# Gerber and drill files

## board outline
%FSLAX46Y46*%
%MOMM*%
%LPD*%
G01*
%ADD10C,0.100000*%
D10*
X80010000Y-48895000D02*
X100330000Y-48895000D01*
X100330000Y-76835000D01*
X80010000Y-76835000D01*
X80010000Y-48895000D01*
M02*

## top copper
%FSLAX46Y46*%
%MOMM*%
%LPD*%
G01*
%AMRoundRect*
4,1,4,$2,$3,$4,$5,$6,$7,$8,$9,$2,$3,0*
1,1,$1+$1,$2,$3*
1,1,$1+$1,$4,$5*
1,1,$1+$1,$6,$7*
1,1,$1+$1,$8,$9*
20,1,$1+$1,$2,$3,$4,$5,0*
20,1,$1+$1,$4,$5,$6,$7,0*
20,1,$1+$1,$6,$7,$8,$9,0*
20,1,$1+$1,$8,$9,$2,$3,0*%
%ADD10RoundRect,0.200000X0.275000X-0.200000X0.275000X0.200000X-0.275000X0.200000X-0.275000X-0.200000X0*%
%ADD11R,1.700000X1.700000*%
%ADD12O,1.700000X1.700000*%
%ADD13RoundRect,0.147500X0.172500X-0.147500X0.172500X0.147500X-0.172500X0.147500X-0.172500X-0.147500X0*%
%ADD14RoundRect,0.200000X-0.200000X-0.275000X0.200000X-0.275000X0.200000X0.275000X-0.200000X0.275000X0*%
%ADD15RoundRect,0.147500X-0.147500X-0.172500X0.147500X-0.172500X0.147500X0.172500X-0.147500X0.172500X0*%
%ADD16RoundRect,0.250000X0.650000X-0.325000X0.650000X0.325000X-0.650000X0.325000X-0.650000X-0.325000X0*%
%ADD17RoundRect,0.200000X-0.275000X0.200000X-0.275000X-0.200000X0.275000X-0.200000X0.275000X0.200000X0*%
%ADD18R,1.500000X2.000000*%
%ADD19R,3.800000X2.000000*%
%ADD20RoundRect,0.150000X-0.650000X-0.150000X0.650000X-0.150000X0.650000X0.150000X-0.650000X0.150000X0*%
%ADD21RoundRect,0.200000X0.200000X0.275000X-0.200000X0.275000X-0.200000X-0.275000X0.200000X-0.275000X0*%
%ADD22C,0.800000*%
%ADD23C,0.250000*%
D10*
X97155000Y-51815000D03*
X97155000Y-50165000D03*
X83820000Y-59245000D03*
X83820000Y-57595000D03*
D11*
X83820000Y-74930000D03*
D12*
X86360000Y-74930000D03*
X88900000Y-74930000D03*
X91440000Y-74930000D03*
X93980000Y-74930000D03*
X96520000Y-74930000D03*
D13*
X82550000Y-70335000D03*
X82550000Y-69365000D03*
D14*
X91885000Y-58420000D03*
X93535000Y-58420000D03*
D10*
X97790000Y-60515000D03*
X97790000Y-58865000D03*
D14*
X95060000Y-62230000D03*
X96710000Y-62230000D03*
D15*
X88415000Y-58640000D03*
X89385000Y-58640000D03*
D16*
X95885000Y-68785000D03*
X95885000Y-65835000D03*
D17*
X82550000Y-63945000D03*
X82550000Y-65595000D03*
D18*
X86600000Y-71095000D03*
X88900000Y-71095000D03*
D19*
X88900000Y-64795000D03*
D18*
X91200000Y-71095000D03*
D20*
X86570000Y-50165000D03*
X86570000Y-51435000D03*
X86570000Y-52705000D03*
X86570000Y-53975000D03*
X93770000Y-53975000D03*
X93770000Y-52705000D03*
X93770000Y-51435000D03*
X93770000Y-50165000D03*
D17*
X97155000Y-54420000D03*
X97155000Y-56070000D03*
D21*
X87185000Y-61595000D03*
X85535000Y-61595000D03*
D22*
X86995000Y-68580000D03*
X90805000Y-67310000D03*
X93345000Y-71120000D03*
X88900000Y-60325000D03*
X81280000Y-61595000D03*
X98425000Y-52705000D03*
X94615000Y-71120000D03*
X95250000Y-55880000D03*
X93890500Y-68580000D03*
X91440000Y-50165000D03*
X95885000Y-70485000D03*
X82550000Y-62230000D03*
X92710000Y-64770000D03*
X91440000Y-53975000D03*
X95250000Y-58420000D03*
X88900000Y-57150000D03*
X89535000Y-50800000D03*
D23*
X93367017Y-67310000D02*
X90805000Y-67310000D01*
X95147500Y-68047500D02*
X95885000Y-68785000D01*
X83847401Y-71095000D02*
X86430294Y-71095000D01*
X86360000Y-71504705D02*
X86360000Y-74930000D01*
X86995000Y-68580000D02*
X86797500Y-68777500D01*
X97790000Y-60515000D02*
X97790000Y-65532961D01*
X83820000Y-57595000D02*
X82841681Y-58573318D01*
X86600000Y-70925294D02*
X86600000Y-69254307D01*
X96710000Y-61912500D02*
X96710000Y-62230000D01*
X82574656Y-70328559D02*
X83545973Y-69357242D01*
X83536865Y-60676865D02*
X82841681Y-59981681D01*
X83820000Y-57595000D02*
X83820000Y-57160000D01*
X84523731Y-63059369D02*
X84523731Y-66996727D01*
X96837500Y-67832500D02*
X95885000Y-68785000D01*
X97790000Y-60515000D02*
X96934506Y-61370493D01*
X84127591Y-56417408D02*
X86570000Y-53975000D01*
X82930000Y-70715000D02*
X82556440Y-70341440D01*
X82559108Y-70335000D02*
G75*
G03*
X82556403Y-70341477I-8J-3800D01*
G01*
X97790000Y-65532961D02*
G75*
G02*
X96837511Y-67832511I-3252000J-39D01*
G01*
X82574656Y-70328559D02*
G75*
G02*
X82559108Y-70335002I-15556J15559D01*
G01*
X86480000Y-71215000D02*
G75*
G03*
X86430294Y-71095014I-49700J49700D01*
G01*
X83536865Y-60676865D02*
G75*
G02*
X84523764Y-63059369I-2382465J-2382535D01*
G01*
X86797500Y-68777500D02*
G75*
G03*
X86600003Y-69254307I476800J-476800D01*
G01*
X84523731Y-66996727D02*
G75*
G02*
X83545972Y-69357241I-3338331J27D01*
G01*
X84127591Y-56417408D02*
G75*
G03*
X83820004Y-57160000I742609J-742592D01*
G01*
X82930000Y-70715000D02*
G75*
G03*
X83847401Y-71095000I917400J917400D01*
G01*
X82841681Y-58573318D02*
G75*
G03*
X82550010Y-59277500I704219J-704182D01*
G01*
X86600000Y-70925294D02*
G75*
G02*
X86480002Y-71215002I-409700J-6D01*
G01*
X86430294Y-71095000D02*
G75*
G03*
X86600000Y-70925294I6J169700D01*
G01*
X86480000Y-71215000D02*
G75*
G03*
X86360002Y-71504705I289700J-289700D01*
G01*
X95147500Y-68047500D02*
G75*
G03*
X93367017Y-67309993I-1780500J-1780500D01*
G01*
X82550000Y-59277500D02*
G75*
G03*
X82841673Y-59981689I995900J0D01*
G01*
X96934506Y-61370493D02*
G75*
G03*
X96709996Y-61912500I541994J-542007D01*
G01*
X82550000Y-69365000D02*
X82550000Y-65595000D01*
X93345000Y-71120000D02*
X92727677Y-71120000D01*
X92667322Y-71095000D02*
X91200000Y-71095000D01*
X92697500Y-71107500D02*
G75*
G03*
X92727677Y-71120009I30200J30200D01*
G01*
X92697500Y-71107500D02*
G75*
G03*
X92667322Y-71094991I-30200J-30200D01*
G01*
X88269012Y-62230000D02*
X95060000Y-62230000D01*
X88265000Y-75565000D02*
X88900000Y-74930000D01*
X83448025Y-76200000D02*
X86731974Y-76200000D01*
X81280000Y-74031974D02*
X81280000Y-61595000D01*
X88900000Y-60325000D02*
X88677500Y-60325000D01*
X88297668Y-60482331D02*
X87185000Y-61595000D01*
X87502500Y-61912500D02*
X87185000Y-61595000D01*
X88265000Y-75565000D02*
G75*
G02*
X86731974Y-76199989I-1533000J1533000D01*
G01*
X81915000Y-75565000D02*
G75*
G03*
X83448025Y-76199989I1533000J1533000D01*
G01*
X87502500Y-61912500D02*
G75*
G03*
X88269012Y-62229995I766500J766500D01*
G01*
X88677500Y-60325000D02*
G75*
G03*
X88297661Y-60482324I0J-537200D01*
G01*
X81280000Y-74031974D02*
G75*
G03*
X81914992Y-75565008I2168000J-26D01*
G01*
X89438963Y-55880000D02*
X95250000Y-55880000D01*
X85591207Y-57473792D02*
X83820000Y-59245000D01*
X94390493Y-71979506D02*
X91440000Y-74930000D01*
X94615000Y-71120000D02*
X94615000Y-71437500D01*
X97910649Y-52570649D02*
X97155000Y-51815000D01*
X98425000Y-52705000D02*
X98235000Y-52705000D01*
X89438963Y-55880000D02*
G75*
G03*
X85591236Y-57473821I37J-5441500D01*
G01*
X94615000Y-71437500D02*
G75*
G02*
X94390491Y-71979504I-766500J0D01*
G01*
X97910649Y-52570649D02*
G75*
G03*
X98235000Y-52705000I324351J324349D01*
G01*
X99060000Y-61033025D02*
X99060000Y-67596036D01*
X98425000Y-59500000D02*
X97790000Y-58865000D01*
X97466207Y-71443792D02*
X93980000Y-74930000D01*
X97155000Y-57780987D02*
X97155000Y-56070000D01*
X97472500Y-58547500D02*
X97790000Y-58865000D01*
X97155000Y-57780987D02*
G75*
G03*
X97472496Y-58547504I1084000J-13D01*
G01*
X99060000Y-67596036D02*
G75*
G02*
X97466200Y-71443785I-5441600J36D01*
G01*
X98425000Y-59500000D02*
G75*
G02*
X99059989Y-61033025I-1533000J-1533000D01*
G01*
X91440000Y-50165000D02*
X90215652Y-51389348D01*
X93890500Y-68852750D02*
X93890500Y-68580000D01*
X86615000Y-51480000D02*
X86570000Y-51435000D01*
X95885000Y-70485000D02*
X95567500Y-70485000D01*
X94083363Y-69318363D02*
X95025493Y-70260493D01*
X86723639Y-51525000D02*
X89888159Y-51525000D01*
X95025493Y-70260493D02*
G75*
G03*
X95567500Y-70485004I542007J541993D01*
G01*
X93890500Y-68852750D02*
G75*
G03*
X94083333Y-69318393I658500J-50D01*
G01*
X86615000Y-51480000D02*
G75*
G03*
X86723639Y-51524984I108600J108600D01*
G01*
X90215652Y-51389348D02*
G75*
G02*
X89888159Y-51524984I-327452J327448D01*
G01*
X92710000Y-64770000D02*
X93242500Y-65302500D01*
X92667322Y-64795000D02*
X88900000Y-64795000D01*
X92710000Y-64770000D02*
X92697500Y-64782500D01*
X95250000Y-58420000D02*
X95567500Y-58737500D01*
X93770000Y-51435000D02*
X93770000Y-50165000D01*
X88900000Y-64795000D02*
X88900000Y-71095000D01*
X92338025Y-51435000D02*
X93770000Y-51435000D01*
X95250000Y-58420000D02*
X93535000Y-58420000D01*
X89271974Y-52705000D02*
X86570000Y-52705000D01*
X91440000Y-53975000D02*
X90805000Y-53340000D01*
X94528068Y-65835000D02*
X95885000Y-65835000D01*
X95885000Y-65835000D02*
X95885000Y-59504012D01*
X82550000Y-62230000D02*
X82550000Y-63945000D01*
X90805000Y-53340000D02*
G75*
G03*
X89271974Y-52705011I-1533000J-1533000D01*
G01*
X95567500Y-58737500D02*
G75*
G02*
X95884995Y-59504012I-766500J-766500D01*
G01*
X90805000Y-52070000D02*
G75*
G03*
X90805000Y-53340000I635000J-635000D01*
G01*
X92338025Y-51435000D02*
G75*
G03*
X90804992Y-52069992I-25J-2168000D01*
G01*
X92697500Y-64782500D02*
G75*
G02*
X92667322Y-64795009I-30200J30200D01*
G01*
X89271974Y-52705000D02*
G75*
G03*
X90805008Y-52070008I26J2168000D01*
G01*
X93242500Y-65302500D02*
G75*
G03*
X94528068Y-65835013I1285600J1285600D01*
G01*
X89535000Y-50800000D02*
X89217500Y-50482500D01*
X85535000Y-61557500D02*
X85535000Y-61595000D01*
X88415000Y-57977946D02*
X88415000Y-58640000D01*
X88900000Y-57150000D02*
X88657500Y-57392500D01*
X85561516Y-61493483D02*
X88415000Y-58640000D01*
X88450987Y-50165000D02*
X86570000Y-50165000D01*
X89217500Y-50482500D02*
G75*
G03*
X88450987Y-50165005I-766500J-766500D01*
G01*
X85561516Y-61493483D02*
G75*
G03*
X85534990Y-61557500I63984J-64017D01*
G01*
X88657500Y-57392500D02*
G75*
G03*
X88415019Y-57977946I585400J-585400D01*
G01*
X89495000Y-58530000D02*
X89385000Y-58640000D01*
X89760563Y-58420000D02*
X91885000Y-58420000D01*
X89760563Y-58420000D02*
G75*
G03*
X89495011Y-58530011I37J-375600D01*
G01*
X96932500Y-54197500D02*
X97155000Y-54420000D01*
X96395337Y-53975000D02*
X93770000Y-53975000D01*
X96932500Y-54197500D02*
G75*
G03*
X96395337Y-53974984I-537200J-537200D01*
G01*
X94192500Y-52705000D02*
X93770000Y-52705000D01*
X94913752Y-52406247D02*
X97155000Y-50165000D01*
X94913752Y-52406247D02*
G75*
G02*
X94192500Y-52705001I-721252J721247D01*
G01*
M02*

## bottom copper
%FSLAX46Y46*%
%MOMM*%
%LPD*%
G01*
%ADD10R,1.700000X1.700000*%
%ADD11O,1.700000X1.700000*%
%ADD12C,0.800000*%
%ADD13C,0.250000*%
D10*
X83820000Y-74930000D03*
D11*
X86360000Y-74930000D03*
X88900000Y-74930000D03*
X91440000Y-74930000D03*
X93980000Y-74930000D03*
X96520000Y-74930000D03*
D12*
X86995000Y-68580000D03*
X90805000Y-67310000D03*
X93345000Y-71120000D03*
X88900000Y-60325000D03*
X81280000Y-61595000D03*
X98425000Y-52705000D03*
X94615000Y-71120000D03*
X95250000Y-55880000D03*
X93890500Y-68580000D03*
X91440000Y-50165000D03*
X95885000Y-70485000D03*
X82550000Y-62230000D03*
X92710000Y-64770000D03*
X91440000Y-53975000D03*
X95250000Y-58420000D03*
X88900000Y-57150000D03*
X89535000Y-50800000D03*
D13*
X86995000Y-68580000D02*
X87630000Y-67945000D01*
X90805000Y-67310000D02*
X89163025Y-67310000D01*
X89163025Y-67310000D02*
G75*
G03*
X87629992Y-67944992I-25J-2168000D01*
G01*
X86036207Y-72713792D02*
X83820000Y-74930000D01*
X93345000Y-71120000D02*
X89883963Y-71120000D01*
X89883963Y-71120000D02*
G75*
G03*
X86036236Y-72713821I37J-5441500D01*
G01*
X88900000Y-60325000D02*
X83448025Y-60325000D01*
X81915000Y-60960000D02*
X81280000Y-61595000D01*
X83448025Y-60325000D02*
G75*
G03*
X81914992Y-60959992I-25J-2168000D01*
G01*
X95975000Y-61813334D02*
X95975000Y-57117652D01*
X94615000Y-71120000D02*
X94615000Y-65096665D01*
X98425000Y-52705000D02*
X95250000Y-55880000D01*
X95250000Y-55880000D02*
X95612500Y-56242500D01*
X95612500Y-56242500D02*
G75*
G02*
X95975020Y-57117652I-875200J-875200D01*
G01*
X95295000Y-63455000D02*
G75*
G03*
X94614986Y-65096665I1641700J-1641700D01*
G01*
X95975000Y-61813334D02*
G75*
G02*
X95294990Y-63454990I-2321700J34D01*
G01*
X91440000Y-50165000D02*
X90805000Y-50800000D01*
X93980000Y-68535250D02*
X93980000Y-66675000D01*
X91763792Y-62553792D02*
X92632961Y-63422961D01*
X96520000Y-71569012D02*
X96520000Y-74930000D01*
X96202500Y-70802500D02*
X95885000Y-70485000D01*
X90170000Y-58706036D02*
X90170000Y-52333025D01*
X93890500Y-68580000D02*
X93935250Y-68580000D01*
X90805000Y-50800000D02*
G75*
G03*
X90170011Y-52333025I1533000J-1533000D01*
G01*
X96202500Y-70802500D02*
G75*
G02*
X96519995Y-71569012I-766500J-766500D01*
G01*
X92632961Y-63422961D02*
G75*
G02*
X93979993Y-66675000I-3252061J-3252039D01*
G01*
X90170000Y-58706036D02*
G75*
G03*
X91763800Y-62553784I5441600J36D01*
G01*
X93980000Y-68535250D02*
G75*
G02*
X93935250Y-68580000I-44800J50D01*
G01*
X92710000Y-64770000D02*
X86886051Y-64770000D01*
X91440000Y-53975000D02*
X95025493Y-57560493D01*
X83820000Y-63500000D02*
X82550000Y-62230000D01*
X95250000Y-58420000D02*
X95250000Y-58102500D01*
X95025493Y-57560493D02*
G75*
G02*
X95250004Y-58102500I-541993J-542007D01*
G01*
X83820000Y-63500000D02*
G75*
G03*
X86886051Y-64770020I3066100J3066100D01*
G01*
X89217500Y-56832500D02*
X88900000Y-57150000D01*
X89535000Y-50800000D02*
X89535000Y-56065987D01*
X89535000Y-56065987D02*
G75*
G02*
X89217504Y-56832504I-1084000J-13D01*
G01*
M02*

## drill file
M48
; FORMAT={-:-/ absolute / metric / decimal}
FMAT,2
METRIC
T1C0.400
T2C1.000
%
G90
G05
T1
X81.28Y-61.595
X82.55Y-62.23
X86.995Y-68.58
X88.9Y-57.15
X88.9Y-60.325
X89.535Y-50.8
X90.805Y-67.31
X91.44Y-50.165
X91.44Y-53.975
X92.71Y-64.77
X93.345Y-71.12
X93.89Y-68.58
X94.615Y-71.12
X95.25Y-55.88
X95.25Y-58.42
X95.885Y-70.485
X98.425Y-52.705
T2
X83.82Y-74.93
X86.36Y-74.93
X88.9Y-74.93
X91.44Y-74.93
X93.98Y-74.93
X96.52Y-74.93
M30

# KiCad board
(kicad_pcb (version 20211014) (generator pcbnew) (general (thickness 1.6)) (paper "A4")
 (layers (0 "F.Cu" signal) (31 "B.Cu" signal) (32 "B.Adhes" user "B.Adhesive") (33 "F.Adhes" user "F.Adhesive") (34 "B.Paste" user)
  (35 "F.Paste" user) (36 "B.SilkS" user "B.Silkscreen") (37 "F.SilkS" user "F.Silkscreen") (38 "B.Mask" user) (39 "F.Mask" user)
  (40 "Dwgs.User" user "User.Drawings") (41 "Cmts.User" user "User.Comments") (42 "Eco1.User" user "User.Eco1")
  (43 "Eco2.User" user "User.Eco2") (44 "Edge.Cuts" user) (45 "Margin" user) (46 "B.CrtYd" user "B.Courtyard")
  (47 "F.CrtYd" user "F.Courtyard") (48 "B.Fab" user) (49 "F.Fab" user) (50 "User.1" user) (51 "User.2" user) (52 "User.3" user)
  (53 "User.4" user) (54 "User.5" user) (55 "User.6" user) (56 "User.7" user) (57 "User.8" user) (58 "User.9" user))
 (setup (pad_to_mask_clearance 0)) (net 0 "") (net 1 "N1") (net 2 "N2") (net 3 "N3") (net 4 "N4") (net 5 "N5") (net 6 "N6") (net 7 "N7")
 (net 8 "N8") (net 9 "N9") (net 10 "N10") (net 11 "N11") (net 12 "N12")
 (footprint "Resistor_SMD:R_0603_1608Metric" (layer "F.Cu") (at 97.155 50.99 90)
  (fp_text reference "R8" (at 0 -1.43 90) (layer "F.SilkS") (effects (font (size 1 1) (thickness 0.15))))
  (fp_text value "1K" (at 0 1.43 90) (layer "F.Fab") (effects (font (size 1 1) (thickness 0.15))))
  (pad "1" smd roundrect (at -0.825 0 90) (size 0.8 0.95) (layers "F.Cu" "F.Paste" "F.Mask") (roundrect_rratio 0.25) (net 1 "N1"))
  (pad "2" smd roundrect (at 0.825 0 90) (size 0.8 0.95) (layers "F.Cu" "F.Paste" "F.Mask") (roundrect_rratio 0.25) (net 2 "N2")))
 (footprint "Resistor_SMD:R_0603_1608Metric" (layer "F.Cu") (at 83.82 58.42 90)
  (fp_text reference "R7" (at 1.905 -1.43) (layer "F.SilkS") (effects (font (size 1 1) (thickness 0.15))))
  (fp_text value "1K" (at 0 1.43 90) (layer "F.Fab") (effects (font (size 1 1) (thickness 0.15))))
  (pad "1" smd roundrect (at -0.825 0 90) (size 0.8 0.95) (layers "F.Cu" "F.Paste" "F.Mask") (roundrect_rratio 0.25) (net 1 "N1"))
  (pad "2" smd roundrect (at 0.825 0 90) (size 0.8 0.95) (layers "F.Cu" "F.Paste" "F.Mask") (roundrect_rratio 0.25) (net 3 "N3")))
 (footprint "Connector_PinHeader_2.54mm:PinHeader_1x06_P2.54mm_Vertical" (layer "F.Cu") (at 83.82 74.93 90)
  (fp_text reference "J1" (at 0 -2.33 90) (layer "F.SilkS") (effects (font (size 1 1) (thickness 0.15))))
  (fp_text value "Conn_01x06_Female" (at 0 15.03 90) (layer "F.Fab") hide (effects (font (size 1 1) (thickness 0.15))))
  (pad "1" thru_hole rect (at 0 0 90) (size 1.7 1.7) (drill 1) (layers *.Cu *.Mask) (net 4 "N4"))
  (pad "2" thru_hole oval (at 0 2.54 90) (size 1.7 1.7) (drill 1) (layers *.Cu *.Mask) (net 3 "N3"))
  (pad "3" thru_hole oval (at 0 5.08 90) (size 1.7 1.7) (drill 1) (layers *.Cu *.Mask) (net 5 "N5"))
  (pad "4" thru_hole oval (at 0 7.62 90) (size 1.7 1.7) (drill 1) (layers *.Cu *.Mask) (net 1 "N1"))
  (pad "5" thru_hole oval (at 0 10.16 90) (size 1.7 1.7) (drill 1) (layers *.Cu *.Mask) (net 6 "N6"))
  (pad "6" thru_hole oval (at 0 12.7 90) (size 1.7 1.7) (drill 1) (layers *.Cu *.Mask) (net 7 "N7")))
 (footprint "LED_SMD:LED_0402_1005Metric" (layer "F.Cu") (at 82.55 69.85 90)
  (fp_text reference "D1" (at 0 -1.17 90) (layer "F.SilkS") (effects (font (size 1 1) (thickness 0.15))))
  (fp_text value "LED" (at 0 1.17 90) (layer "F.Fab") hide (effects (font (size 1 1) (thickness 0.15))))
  (pad "1" smd roundrect (at -0.485 0 90) (size 0.59 0.64) (layers "F.Cu" "F.Paste" "F.Mask") (roundrect_rratio 0.25) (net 3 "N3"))
  (pad "2" smd roundrect (at 0.485 0 90) (size 0.59 0.64) (layers "F.Cu" "F.Paste" "F.Mask") (roundrect_rratio 0.25) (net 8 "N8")))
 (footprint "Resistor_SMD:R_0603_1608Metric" (layer "F.Cu") (at 92.71 58.42)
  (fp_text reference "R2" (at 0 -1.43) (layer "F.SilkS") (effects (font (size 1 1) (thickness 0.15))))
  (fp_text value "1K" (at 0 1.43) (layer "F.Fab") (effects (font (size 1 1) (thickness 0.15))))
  (pad "1" smd roundrect (at -0.825 0) (size 0.8 0.95) (layers "F.Cu" "F.Paste" "F.Mask") (roundrect_rratio 0.25) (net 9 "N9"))
  (pad "2" smd roundrect (at 0.825 0) (size 0.8 0.95) (layers "F.Cu" "F.Paste" "F.Mask") (roundrect_rratio 0.25) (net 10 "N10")))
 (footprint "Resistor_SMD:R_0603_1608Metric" (layer "F.Cu") (at 97.79 59.69 90)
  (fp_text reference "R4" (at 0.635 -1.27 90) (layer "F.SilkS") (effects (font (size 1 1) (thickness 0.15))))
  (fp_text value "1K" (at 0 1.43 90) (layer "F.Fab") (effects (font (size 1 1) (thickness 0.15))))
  (pad "1" smd roundrect (at -0.825 0 90) (size 0.8 0.95) (layers "F.Cu" "F.Paste" "F.Mask") (roundrect_rratio 0.25) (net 3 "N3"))
  (pad "2" smd roundrect (at 0.825 0 90) (size 0.8 0.95) (layers "F.Cu" "F.Paste" "F.Mask") (roundrect_rratio 0.25) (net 6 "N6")))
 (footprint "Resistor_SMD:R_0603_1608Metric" (layer "F.Cu") (at 95.885 62.23)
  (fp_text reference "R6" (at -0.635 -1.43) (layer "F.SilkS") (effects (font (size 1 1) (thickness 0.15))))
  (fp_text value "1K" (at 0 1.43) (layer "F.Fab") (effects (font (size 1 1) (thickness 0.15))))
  (pad "1" smd roundrect (at -0.825 0) (size 0.8 0.95) (layers "F.Cu" "F.Paste" "F.Mask") (roundrect_rratio 0.25) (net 5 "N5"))
  (pad "2" smd roundrect (at 0.825 0) (size 0.8 0.95) (layers "F.Cu" "F.Paste" "F.Mask") (roundrect_rratio 0.25) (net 3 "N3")))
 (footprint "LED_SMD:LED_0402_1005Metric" (layer "F.Cu") (at 88.9 58.64)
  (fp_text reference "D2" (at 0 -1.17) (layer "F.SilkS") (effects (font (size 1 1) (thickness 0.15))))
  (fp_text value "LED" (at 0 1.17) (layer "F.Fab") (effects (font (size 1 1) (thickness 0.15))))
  (pad "1" smd roundrect (at -0.485 0) (size 0.59 0.64) (layers "F.Cu" "F.Paste" "F.Mask") (roundrect_rratio 0.25) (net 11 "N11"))
  (pad "2" smd roundrect (at 0.485 0) (size 0.59 0.64) (layers "F.Cu" "F.Paste" "F.Mask") (roundrect_rratio 0.25) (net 9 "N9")))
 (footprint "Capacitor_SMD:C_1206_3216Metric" (layer "F.Cu") (at 95.885 67.31 90)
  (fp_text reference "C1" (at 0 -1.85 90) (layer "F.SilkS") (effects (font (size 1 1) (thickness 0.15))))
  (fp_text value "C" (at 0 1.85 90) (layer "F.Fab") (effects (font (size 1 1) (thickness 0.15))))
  (pad "1" smd roundrect (at -1.475 0 90) (size 1.15 1.8) (layers "F.Cu" "F.Paste" "F.Mask") (roundrect_rratio 0.2173913043) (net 3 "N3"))
  (pad "2" smd roundrect (at 1.475 0 90) (size 1.15 1.8) (layers "F.Cu" "F.Paste" "F.Mask") (roundrect_rratio 0.2173913043) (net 10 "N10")))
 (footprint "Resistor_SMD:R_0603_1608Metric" (layer "F.Cu") (at 82.55 64.77 -90)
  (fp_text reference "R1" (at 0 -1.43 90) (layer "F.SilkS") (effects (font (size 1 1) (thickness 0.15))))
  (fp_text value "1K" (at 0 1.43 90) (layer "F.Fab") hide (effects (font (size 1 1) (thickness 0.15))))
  (pad "1" smd roundrect (at -0.825 0 270) (size 0.8 0.95) (layers "F.Cu" "F.Paste" "F.Mask") (roundrect_rratio 0.25) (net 10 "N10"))
  (pad "2" smd roundrect (at 0.825 0 270) (size 0.8 0.95) (layers "F.Cu" "F.Paste" "F.Mask") (roundrect_rratio 0.25) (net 8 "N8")))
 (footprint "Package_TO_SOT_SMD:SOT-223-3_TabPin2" (layer "F.Cu") (at 88.9 67.945 90)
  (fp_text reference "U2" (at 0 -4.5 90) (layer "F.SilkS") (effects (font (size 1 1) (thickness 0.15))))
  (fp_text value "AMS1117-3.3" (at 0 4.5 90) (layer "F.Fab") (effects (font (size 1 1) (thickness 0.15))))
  (pad "1" smd rect (at -3.15 -2.3 90) (size 2 1.5) (layers "F.Cu" "F.Paste" "F.Mask") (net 3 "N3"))
  (pad "2" smd rect (at -3.15 0 90) (size 2 1.5) (layers "F.Cu" "F.Paste" "F.Mask") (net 10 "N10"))
  (pad "2" smd rect (at 3.15 0 90) (size 2 3.8) (layers "F.Cu" "F.Paste" "F.Mask") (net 10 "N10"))
  (pad "3" smd rect (at -3.15 2.3 90) (size 2 1.5) (layers "F.Cu" "F.Paste" "F.Mask") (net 4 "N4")))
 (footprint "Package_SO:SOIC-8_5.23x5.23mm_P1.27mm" (layer "F.Cu") (at 90.17 52.07)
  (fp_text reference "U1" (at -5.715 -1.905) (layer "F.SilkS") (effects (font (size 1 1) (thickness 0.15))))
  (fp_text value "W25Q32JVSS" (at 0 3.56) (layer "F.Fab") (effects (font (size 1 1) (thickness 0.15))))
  (pad "1" smd roundrect (at -3.6 -1.905) (size 1.6 0.6) (layers "F.Cu" "F.Paste" "F.Mask") (roundrect_rratio 0.25) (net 11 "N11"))
  (pad "2" smd roundrect (at -3.6 -0.635) (size 1.6 0.6) (layers "F.Cu" "F.Paste" "F.Mask") (roundrect_rratio 0.25) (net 7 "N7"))
  (pad "3" smd roundrect (at -3.6 0.635) (size 1.6 0.6) (layers "F.Cu" "F.Paste" "F.Mask") (roundrect_rratio 0.25) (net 10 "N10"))
  (pad "4" smd roundrect (at -3.6 1.905) (size 1.6 0.6) (layers "F.Cu" "F.Paste" "F.Mask") (roundrect_rratio 0.25) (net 3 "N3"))
  (pad "5" smd roundrect (at 3.6 1.905) (size 1.6 0.6) (layers "F.Cu" "F.Paste" "F.Mask") (roundrect_rratio 0.25) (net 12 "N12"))
  (pad "6" smd roundrect (at 3.6 0.635) (size 1.6 0.6) (layers "F.Cu" "F.Paste" "F.Mask") (roundrect_rratio 0.25) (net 2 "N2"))
  (pad "7" smd roundrect (at 3.6 -0.635) (size 1.6 0.6) (layers "F.Cu" "F.Paste" "F.Mask") (roundrect_rratio 0.25) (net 10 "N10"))
  (pad "8" smd roundrect (at 3.6 -1.905) (size 1.6 0.6) (layers "F.Cu" "F.Paste" "F.Mask") (roundrect_rratio 0.25) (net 10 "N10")))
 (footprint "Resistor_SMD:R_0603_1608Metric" (layer "F.Cu") (at 97.155 55.245 -90)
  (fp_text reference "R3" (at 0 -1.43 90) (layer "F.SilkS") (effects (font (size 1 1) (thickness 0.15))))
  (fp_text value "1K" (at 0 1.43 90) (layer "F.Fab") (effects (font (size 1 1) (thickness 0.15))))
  (pad "1" smd roundrect (at -0.825 0 270) (size 0.8 0.95) (layers "F.Cu" "F.Paste" "F.Mask") (roundrect_rratio 0.25) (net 12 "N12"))
  (pad "2" smd roundrect (at 0.825 0 270) (size 0.8 0.95) (layers "F.Cu" "F.Paste" "F.Mask") (roundrect_rratio 0.25) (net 6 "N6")))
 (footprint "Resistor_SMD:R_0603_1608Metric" (layer "F.Cu") (at 86.36 61.595 180)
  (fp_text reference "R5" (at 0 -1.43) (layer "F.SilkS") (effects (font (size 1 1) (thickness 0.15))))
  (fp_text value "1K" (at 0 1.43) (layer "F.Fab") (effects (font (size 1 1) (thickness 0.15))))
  (pad "1" smd roundrect (at -0.825 0 180) (size 0.8 0.95) (layers "F.Cu" "F.Paste" "F.Mask") (roundrect_rratio 0.25) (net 5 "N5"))
  (pad "2" smd roundrect (at 0.825 0 180) (size 0.8 0.95) (layers "F.Cu" "F.Paste" "F.Mask") (roundrect_rratio 0.25) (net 11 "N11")))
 (gr_rect (start 80.01 48.895) (end 100.33 76.835) (layer "Edge.Cuts") (width 0.1) (fill none))
 (segment (start 93.367017 67.31) (end 90.805 67.31) (width 0.25) (layer "F.Cu") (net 3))
 (segment (start 95.1475 68.0475) (end 95.885 68.785) (width 0.25) (layer "F.Cu") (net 3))
 (segment (start 83.847401 71.095) (end 86.430294 71.095) (width 0.25) (layer "F.Cu") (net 3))
 (segment (start 86.36 71.504705) (end 86.36 74.93) (width 0.25) (layer "F.Cu") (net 3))
 (segment (start 86.995 68.58) (end 86.7975 68.7775) (width 0.25) (layer "F.Cu") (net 3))
 (segment (start 97.79 60.515) (end 97.79 65.532961) (width 0.25) (layer "F.Cu") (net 3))
 (segment (start 83.82 57.595) (end 82.841681 58.573318) (width 0.25) (layer "F.Cu") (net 3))
 (segment (start 86.6 70.925294) (end 86.6 69.254307) (width 0.25) (layer "F.Cu") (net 3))
 (segment (start 96.71 61.9125) (end 96.71 62.23) (width 0.25) (layer "F.Cu") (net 3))
 (segment (start 82.574656 70.328559) (end 83.545973 69.357242) (width 0.25) (layer "F.Cu") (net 3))
 (segment (start 83.536865 60.676865) (end 82.841681 59.981681) (width 0.25) (layer "F.Cu") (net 3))
 (segment (start 83.82 57.595) (end 83.82 57.16) (width 0.25) (layer "F.Cu") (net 3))
 (segment (start 84.523731 63.059369) (end 84.523731 66.996727) (width 0.25) (layer "F.Cu") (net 3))
 (segment (start 96.8375 67.8325) (end 95.885 68.785) (width 0.25) (layer "F.Cu") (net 3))
 (segment (start 97.79 60.515) (end 96.934506 61.370493) (width 0.25) (layer "F.Cu") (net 3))
 (segment (start 84.127591 56.417408) (end 86.57 53.975) (width 0.25) (layer "F.Cu") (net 3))
 (segment (start 82.93 70.715) (end 82.55644 70.34144) (width 0.25) (layer "F.Cu") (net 3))
 (via (at 86.995 68.58) (size 0.8) (drill 0.4) (layers "F.Cu" "B.Cu") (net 3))
 (via (at 90.805 67.31) (size 0.8) (drill 0.4) (layers "F.Cu" "B.Cu") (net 3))
 (arc (start 82.559108 70.335) (mid 82.555622 70.337328) (end 82.55644 70.34144) (width 0.25) (layer "F.Cu") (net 3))
 (arc (start 97.79 65.532961) (mid 97.542453 66.777462) (end 96.8375 67.8325) (width 0.25) (layer "F.Cu") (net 3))
 (arc (start 82.574656 70.328559) (mid 82.567522 70.333326) (end 82.559108 70.335) (width 0.25) (layer "F.Cu") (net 3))
 (arc (start 86.48 71.215) (mid 86.495237 71.138393) (end 86.430294 71.095) (width 0.25) (layer "F.Cu") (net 3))
 (arc (start 83.536865 60.676865) (mid 84.267252 61.769967) (end 84.523731 63.059369) (width 0.25) (layer "F.Cu") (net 3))
 (arc (start 86.7975 68.7775) (mid 86.651328 68.99626) (end 86.6 69.254307) (width 0.25) (layer "F.Cu") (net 3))
 (arc (start 84.523731 66.996727) (mid 84.269619 68.274228) (end 83.545973 69.357242) (width 0.25) (layer "F.Cu") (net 3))
 (arc (start 84.127591 56.417408) (mid 83.89994 56.758112) (end 83.82 57.16) (width 0.25) (layer "F.Cu") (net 3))
 (arc (start 82.93 70.715) (mid 83.350907 70.996241) (end 83.847401 71.095) (width 0.25) (layer "F.Cu") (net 3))
 (arc (start 82.841681 58.573318) (mid 82.625805 58.896399) (end 82.55 59.2775) (width 0.25) (layer "F.Cu") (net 3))
 (arc (start 86.6 70.925294) (mid 86.568813 71.082081) (end 86.48 71.215) (width 0.25) (layer "F.Cu") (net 3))
 (arc (start 86.430294 71.095) (mid 86.550294 71.045294) (end 86.6 70.925294) (width 0.25) (layer "F.Cu") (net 3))
 (arc (start 86.48 71.215) (mid 86.391186 71.347917) (end 86.36 71.504705) (width 0.25) (layer "F.Cu") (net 3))
 (arc (start 95.1475 68.0475) (mid 94.330607 67.50167) (end 93.367017 67.31) (width 0.25) (layer "F.Cu") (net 3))
 (arc (start 82.55 59.2775) (mid 82.625805 59.6586) (end 82.841681 59.981681) (width 0.25) (layer "F.Cu") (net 3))
 (arc (start 96.934506 61.370493) (mid 96.768347 61.619168) (end 96.71 61.9125) (width 0.25) (layer "F.Cu") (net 3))
 (segment (start 86.995 68.58) (end 87.63 67.945) (width 0.25) (layer "B.Cu") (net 3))
 (segment (start 90.805 67.31) (end 89.163025 67.31) (width 0.25) (layer "B.Cu") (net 3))
 (arc (start 89.163025 67.31) (mid 88.333357 67.475031) (end 87.63 67.945) (width 0.25) (layer "B.Cu") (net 3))
 (segment (start 82.55 69.365) (end 82.55 65.595) (width 0.25) (layer "F.Cu") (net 8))
 (segment (start 93.345 71.12) (end 92.727677 71.12) (width 0.25) (layer "F.Cu") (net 4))
 (segment (start 92.667322 71.095) (end 91.2 71.095) (width 0.25) (layer "F.Cu") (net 4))
 (via (at 93.345 71.12) (size 0.8) (drill 0.4) (layers "F.Cu" "B.Cu") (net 4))
 (arc (start 92.6975 71.1075) (mid 92.711345 71.116751) (end 92.727677 71.12) (width 0.25) (layer "F.Cu") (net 4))
 (arc (start 92.6975 71.1075) (mid 92.683654 71.098248) (end 92.667322 71.095) (width 0.25) (layer "F.Cu") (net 4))
 (segment (start 86.036207 72.713792) (end 83.82 74.93) (width 0.25) (layer "B.Cu") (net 4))
 (segment (start 93.345 71.12) (end 89.883963 71.12) (width 0.25) (layer "B.Cu") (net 4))
 (arc (start 89.883963 71.12) (mid 87.801572 71.534213) (end 86.036207 72.713792) (width 0.25) (layer "B.Cu") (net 4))
 (segment (start 88.269012 62.23) (end 95.06 62.23) (width 0.25) (layer "F.Cu") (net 5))
 (segment (start 88.265 75.565) (end 88.9 74.93) (width 0.25) (layer "F.Cu") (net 5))
 (segment (start 83.448025 76.2) (end 86.731974 76.2) (width 0.25) (layer "F.Cu") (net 5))
 (segment (start 81.28 74.031974) (end 81.28 61.595) (width 0.25) (layer "F.Cu") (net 5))
 (segment (start 88.9 60.325) (end 88.6775 60.325) (width 0.25) (layer "F.Cu") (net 5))
 (segment (start 88.297668 60.482331) (end 87.185 61.595) (width 0.25) (layer "F.Cu") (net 5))
 (segment (start 87.5025 61.9125) (end 87.185 61.595) (width 0.25) (layer "F.Cu") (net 5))
 (via (at 88.9 60.325) (size 0.8) (drill 0.4) (layers "F.Cu" "B.Cu") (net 5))
 (via (at 81.28 61.595) (size 0.8) (drill 0.4) (layers "F.Cu" "B.Cu") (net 5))
 (arc (start 88.265 75.565) (mid 87.561641 76.034968) (end 86.731974 76.2) (width 0.25) (layer "F.Cu") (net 5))
 (arc (start 81.915 75.565) (mid 82.618357 76.034968) (end 83.448025 76.2) (width 0.25) (layer "F.Cu") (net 5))
 (arc (start 87.5025 61.9125) (mid 87.854178 62.147484) (end 88.269012 62.23) (width 0.25) (layer "F.Cu") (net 5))
 (arc (start 88.6775 60.325) (mid 88.471936 60.365888) (end 88.297668 60.482331) (width 0.25) (layer "F.Cu") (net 5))
 (arc (start 81.28 74.031974) (mid 81.445031 74.861641) (end 81.915 75.565) (width 0.25) (layer "F.Cu") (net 5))
 (segment (start 88.9 60.325) (end 83.448025 60.325) (width 0.25) (layer "B.Cu") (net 5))
 (segment (start 81.915 60.96) (end 81.28 61.595) (width 0.25) (layer "B.Cu") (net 5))
 (arc (start 83.448025 60.325) (mid 82.618357 60.490031) (end 81.915 60.96) (width 0.25) (layer "B.Cu") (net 5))
 (segment (start 89.438963 55.88) (end 95.25 55.88) (width 0.25) (layer "F.Cu") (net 1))
 (segment (start 85.591207 57.473792) (end 83.82 59.245) (width 0.25) (layer "F.Cu") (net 1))
 (segment (start 94.390493 71.979506) (end 91.44 74.93) (width 0.25) (layer "F.Cu") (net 1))
 (segment (start 94.615 71.12) (end 94.615 71.4375) (width 0.25) (layer "F.Cu") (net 1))
 (segment (start 97.910649 52.570649) (end 97.155 51.815) (width 0.25) (layer "F.Cu") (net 1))
 (segment (start 98.425 52.705) (end 98.235 52.705) (width 0.25) (layer "F.Cu") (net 1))
 (via (at 98.425 52.705) (size 0.8) (drill 0.4) (layers "F.Cu" "B.Cu") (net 1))
 (via (at 94.615 71.12) (size 0.8) (drill 0.4) (layers "F.Cu" "B.Cu") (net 1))
 (via (at 95.25 55.88) (size 0.8) (drill 0.4) (layers "F.Cu" "B.Cu") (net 1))
 (arc (start 89.438963 55.88) (mid 87.356572 56.294213) (end 85.591207 57.473792) (width 0.25) (layer "F.Cu") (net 1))
 (arc (start 94.615 71.4375) (mid 94.556652 71.730831) (end 94.390493 71.979506) (width 0.25) (layer "F.Cu") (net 1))
 (arc (start 97.910649 52.570649) (mid 98.059462 52.670083) (end 98.235 52.705) (width 0.25) (layer "F.Cu") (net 1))
 (segment (start 95.975 61.813334) (end 95.975 57.117652) (width 0.25) (layer "B.Cu") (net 1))
 (segment (start 94.615 71.12) (end 94.615 65.096665) (width 0.25) (layer "B.Cu") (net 1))
 (segment (start 98.425 52.705) (end 95.25 55.88) (width 0.25) (layer "B.Cu") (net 1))
 (segment (start 95.25 55.88) (end 95.6125 56.2425) (width 0.25) (layer "B.Cu") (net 1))
 (arc (start 95.6125 56.2425) (mid 95.880789 56.644023) (end 95.975 57.117652) (width 0.25) (layer "B.Cu") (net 1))
 (arc (start 95.295 63.455) (mid 94.791726 64.208202) (end 94.615 65.096665) (width 0.25) (layer "B.Cu") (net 1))
 (arc (start 95.975 61.813334) (mid 95.798273 62.701797) (end 95.295 63.455) (width 0.25) (layer "B.Cu") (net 1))
 (segment (start 99.06 61.033025) (end 99.06 67.596036) (width 0.25) (layer "F.Cu") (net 6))
 (segment (start 98.425 59.5) (end 97.79 58.865) (width 0.25) (layer "F.Cu") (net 6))
 (segment (start 97.466207 71.443792) (end 93.98 74.93) (width 0.25) (layer "F.Cu") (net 6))
 (segment (start 97.155 57.780987) (end 97.155 56.07) (width 0.25) (layer "F.Cu") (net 6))
 (segment (start 97.4725 58.5475) (end 97.79 58.865) (width 0.25) (layer "F.Cu") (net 6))
 (arc (start 97.155 57.780987) (mid 97.237515 58.19582) (end 97.4725 58.5475) (width 0.25) (layer "F.Cu") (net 6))
 (arc (start 99.06 67.596036) (mid 98.645786 69.678426) (end 97.466207 71.443792) (width 0.25) (layer "F.Cu") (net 6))
 (arc (start 98.425 59.5) (mid 98.894968 60.203357) (end 99.06 61.033025) (width 0.25) (layer "F.Cu") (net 6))
 (segment (start 91.44 50.165) (end 90.215652 51.389348) (width 0.25) (layer "F.Cu") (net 7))
 (segment (start 93.8905 68.85275) (end 93.8905 68.58) (width 0.25) (layer "F.Cu") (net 7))
 (segment (start 86.615 51.48) (end 86.57 51.435) (width 0.25) (layer "F.Cu") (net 7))
 (segment (start 95.885 70.485) (end 95.5675 70.485) (width 0.25) (layer "F.Cu") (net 7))
 (segment (start 94.083363 69.318363) (end 95.025493 70.260493) (width 0.25) (layer "F.Cu") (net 7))
 (segment (start 86.723639 51.525) (end 89.888159 51.525) (width 0.25) (layer "F.Cu") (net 7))
 (via (at 93.8905 68.58) (size 0.8) (drill 0.4) (layers "F.Cu" "B.Cu") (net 7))
 (via (at 91.44 50.165) (size 0.8) (drill 0.4) (layers "F.Cu" "B.Cu") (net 7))
 (via (at 95.885 70.485) (size 0.8) (drill 0.4) (layers "F.Cu" "B.Cu") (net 7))
 (arc (start 95.025493 70.260493) (mid 95.274168 70.426652) (end 95.5675 70.485) (width 0.25) (layer "F.Cu") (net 7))
 (arc (start 93.8905 68.85275) (mid 93.940623 69.104738) (end 94.083363 69.318363) (width 0.25) (layer "F.Cu") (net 7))
 (arc (start 86.615 51.48) (mid 86.664844 51.513304) (end 86.723639 51.525) (width 0.25) (layer "F.Cu") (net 7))
 (arc (start 90.215652 51.389348) (mid 90.065397 51.489745) (end 89.888159 51.525) (width 0.25) (layer "F.Cu") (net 7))
 (segment (start 91.44 50.165) (end 90.805 50.8) (width 0.25) (layer "B.Cu") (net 7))
 (segment (start 93.98 68.53525) (end 93.98 66.675) (width 0.25) (layer "B.Cu") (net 7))
 (segment (start 91.763792 62.553792) (end 92.632961 63.422961) (width 0.25) (layer "B.Cu") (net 7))
 (segment (start 96.52 71.569012) (end 96.52 74.93) (width 0.25) (layer "B.Cu") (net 7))
 (segment (start 96.2025 70.8025) (end 95.885 70.485) (width 0.25) (layer "B.Cu") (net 7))
 (segment (start 90.17 58.706036) (end 90.17 52.333025) (width 0.25) (layer "B.Cu") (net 7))
 (segment (start 93.8905 68.58) (end 93.93525 68.58) (width 0.25) (layer "B.Cu") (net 7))
 (arc (start 90.805 50.8) (mid 90.335031 51.503357) (end 90.17 52.333025) (width 0.25) (layer "B.Cu") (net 7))
 (arc (start 96.2025 70.8025) (mid 96.437484 71.154178) (end 96.52 71.569012) (width 0.25) (layer "B.Cu") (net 7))
 (arc (start 92.632961 63.422961) (mid 93.629915 64.915009) (end 93.98 66.675) (width 0.25) (layer "B.Cu") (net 7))
 (arc (start 90.17 58.706036) (mid 90.584213 60.788426) (end 91.763792 62.553792) (width 0.25) (layer "B.Cu") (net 7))
 (arc (start 93.98 68.53525) (mid 93.966893 68.566893) (end 93.93525 68.58) (width 0.25) (layer "B.Cu") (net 7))
 (segment (start 92.71 64.77) (end 93.2425 65.3025) (width 0.25) (layer "F.Cu") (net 10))
 (segment (start 92.667322 64.795) (end 88.9 64.795) (width 0.25) (layer "F.Cu") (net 10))
 (segment (start 92.71 64.77) (end 92.6975 64.7825) (width 0.25) (layer "F.Cu") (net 10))
 (segment (start 95.25 58.42) (end 95.5675 58.7375) (width 0.25) (layer "F.Cu") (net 10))
 (segment (start 93.77 51.435) (end 93.77 50.165) (width 0.25) (layer "F.Cu") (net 10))
 (segment (start 88.9 64.795) (end 88.9 71.095) (width 0.25) (layer "F.Cu") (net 10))
 (segment (start 92.338025 51.435) (end 93.77 51.435) (width 0.25) (layer "F.Cu") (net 10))
 (segment (start 95.25 58.42) (end 93.535 58.42) (width 0.25) (layer "F.Cu") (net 10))
 (segment (start 89.271974 52.705) (end 86.57 52.705) (width 0.25) (layer "F.Cu") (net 10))
 (segment (start 91.44 53.975) (end 90.805 53.34) (width 0.25) (layer "F.Cu") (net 10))
 (segment (start 94.528068 65.835) (end 95.885 65.835) (width 0.25) (layer "F.Cu") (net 10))
 (segment (start 95.885 65.835) (end 95.885 59.504012) (width 0.25) (layer "F.Cu") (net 10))
 (segment (start 82.55 62.23) (end 82.55 63.945) (width 0.25) (layer "F.Cu") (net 10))
 (via (at 82.55 62.23) (size 0.8) (drill 0.4) (layers "F.Cu" "B.Cu") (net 10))
 (via (at 92.71 64.77) (size 0.8) (drill 0.4) (layers "F.Cu" "B.Cu") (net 10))
 (via (at 91.44 53.975) (size 0.8) (drill 0.4) (layers "F.Cu" "B.Cu") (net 10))
 (via (at 95.25 58.42) (size 0.8) (drill 0.4) (layers "F.Cu" "B.Cu") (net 10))
 (arc (start 90.805 53.34) (mid 90.101641 52.870031) (end 89.271974 52.705) (width 0.25) (layer "F.Cu") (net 10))
 (arc (start 95.5675 58.7375) (mid 95.802484 59.089178) (end 95.885 59.504012) (width 0.25) (layer "F.Cu") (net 10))
 (arc (start 90.805 52.07) (mid 90.541974 52.705) (end 90.805 53.34) (width 0.25) (layer "F.Cu") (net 10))
 (arc (start 92.338025 51.435) (mid 91.508357 51.600031) (end 90.805 52.07) (width 0.25) (layer "F.Cu") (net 10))
 (arc (start 92.6975 64.7825) (mid 92.683654 64.791751) (end 92.667322 64.795) (width 0.25) (layer "F.Cu") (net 10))
 (arc (start 89.271974 52.705) (mid 90.101641 52.539968) (end 90.805 52.07) (width 0.25) (layer "F.Cu") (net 10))
 (arc (start 93.2425 65.3025) (mid 93.832323 65.696607) (end 94.528068 65.835) (width 0.25) (layer "F.Cu") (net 10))
 (segment (start 92.71 64.77) (end 86.886051 64.77) (width 0.25) (layer "B.Cu") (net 10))
 (segment (start 91.44 53.975) (end 95.025493 57.560493) (width 0.25) (layer "B.Cu") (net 10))
 (segment (start 83.82 63.5) (end 82.55 62.23) (width 0.25) (layer "B.Cu") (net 10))
 (segment (start 95.25 58.42) (end 95.25 58.1025) (width 0.25) (layer "B.Cu") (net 10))
 (arc (start 95.025493 57.560493) (mid 95.191652 57.809168) (end 95.25 58.1025) (width 0.25) (layer "B.Cu") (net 10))
 (arc (start 83.82 63.5) (mid 85.226716 64.439937) (end 86.886051 64.77) (width 0.25) (layer "B.Cu") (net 10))
 (segment (start 89.535 50.8) (end 89.2175 50.4825) (width 0.25) (layer "F.Cu") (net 11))
 (segment (start 85.535 61.5575) (end 85.535 61.595) (width 0.25) (layer "F.Cu") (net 11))
 (segment (start 88.415 57.977946) (end 88.415 58.64) (width 0.25) (layer "F.Cu") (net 11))
 (segment (start 88.9 57.15) (end 88.6575 57.3925) (width 0.25) (layer "F.Cu") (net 11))
 (segment (start 85.561516 61.493483) (end 88.415 58.64) (width 0.25) (layer "F.Cu") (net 11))
 (segment (start 88.450987 50.165) (end 86.57 50.165) (width 0.25) (layer "F.Cu") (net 11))
 (via (at 88.9 57.15) (size 0.8) (drill 0.4) (layers "F.Cu" "B.Cu") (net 11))
 (via (at 89.535 50.8) (size 0.8) (drill 0.4) (layers "F.Cu" "B.Cu") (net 11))
 (arc (start 89.2175 50.4825) (mid 88.86582 50.247515) (end 88.450987 50.165) (width 0.25) (layer "F.Cu") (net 11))
 (arc (start 85.561516 61.493483) (mid 85.541891 61.522854) (end 85.535 61.5575) (width 0.25) (layer "F.Cu") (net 11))
 (arc (start 88.6575 57.3925) (mid 88.478023 57.661105) (end 88.415 57.977946) (width 0.25) (layer "F.Cu") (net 11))
 (segment (start 89.2175 56.8325) (end 88.9 57.15) (width 0.25) (layer "B.Cu") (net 11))
 (segment (start 89.535 50.8) (end 89.535 56.065987) (width 0.25) (layer "B.Cu") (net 11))
 (arc (start 89.535 56.065987) (mid 89.452484 56.48082) (end 89.2175 56.8325) (width 0.25) (layer "B.Cu") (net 11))
 (segment (start 89.495 58.53) (end 89.385 58.64) (width 0.25) (layer "F.Cu") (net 9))
 (segment (start 89.760563 58.42) (end 91.885 58.42) (width 0.25) (layer "F.Cu") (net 9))
 (arc (start 89.760563 58.42) (mid 89.616841 58.448588) (end 89.495 58.53) (width 0.25) (layer "F.Cu") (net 9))
 (segment (start 96.9325 54.1975) (end 97.155 54.42) (width 0.25) (layer "F.Cu") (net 12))
 (segment (start 96.395337 53.975) (end 93.77 53.975) (width 0.25) (layer "F.Cu") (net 12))
 (arc (start 96.9325 54.1975) (mid 96.686047 54.032825) (end 96.395337 53.975) (width 0.25) (layer "F.Cu") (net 12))
 (segment (start 94.1925 52.705) (end 93.77 52.705) (width 0.25) (layer "F.Cu") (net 2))
 (segment (start 94.913752 52.406247) (end 97.155 50.165) (width 0.25) (layer "F.Cu") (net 2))
 (arc (start 94.913752 52.406247) (mid 94.582838 52.627356) (end 94.1925 52.705) (width 0.25) (layer "F.Cu") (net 2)))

